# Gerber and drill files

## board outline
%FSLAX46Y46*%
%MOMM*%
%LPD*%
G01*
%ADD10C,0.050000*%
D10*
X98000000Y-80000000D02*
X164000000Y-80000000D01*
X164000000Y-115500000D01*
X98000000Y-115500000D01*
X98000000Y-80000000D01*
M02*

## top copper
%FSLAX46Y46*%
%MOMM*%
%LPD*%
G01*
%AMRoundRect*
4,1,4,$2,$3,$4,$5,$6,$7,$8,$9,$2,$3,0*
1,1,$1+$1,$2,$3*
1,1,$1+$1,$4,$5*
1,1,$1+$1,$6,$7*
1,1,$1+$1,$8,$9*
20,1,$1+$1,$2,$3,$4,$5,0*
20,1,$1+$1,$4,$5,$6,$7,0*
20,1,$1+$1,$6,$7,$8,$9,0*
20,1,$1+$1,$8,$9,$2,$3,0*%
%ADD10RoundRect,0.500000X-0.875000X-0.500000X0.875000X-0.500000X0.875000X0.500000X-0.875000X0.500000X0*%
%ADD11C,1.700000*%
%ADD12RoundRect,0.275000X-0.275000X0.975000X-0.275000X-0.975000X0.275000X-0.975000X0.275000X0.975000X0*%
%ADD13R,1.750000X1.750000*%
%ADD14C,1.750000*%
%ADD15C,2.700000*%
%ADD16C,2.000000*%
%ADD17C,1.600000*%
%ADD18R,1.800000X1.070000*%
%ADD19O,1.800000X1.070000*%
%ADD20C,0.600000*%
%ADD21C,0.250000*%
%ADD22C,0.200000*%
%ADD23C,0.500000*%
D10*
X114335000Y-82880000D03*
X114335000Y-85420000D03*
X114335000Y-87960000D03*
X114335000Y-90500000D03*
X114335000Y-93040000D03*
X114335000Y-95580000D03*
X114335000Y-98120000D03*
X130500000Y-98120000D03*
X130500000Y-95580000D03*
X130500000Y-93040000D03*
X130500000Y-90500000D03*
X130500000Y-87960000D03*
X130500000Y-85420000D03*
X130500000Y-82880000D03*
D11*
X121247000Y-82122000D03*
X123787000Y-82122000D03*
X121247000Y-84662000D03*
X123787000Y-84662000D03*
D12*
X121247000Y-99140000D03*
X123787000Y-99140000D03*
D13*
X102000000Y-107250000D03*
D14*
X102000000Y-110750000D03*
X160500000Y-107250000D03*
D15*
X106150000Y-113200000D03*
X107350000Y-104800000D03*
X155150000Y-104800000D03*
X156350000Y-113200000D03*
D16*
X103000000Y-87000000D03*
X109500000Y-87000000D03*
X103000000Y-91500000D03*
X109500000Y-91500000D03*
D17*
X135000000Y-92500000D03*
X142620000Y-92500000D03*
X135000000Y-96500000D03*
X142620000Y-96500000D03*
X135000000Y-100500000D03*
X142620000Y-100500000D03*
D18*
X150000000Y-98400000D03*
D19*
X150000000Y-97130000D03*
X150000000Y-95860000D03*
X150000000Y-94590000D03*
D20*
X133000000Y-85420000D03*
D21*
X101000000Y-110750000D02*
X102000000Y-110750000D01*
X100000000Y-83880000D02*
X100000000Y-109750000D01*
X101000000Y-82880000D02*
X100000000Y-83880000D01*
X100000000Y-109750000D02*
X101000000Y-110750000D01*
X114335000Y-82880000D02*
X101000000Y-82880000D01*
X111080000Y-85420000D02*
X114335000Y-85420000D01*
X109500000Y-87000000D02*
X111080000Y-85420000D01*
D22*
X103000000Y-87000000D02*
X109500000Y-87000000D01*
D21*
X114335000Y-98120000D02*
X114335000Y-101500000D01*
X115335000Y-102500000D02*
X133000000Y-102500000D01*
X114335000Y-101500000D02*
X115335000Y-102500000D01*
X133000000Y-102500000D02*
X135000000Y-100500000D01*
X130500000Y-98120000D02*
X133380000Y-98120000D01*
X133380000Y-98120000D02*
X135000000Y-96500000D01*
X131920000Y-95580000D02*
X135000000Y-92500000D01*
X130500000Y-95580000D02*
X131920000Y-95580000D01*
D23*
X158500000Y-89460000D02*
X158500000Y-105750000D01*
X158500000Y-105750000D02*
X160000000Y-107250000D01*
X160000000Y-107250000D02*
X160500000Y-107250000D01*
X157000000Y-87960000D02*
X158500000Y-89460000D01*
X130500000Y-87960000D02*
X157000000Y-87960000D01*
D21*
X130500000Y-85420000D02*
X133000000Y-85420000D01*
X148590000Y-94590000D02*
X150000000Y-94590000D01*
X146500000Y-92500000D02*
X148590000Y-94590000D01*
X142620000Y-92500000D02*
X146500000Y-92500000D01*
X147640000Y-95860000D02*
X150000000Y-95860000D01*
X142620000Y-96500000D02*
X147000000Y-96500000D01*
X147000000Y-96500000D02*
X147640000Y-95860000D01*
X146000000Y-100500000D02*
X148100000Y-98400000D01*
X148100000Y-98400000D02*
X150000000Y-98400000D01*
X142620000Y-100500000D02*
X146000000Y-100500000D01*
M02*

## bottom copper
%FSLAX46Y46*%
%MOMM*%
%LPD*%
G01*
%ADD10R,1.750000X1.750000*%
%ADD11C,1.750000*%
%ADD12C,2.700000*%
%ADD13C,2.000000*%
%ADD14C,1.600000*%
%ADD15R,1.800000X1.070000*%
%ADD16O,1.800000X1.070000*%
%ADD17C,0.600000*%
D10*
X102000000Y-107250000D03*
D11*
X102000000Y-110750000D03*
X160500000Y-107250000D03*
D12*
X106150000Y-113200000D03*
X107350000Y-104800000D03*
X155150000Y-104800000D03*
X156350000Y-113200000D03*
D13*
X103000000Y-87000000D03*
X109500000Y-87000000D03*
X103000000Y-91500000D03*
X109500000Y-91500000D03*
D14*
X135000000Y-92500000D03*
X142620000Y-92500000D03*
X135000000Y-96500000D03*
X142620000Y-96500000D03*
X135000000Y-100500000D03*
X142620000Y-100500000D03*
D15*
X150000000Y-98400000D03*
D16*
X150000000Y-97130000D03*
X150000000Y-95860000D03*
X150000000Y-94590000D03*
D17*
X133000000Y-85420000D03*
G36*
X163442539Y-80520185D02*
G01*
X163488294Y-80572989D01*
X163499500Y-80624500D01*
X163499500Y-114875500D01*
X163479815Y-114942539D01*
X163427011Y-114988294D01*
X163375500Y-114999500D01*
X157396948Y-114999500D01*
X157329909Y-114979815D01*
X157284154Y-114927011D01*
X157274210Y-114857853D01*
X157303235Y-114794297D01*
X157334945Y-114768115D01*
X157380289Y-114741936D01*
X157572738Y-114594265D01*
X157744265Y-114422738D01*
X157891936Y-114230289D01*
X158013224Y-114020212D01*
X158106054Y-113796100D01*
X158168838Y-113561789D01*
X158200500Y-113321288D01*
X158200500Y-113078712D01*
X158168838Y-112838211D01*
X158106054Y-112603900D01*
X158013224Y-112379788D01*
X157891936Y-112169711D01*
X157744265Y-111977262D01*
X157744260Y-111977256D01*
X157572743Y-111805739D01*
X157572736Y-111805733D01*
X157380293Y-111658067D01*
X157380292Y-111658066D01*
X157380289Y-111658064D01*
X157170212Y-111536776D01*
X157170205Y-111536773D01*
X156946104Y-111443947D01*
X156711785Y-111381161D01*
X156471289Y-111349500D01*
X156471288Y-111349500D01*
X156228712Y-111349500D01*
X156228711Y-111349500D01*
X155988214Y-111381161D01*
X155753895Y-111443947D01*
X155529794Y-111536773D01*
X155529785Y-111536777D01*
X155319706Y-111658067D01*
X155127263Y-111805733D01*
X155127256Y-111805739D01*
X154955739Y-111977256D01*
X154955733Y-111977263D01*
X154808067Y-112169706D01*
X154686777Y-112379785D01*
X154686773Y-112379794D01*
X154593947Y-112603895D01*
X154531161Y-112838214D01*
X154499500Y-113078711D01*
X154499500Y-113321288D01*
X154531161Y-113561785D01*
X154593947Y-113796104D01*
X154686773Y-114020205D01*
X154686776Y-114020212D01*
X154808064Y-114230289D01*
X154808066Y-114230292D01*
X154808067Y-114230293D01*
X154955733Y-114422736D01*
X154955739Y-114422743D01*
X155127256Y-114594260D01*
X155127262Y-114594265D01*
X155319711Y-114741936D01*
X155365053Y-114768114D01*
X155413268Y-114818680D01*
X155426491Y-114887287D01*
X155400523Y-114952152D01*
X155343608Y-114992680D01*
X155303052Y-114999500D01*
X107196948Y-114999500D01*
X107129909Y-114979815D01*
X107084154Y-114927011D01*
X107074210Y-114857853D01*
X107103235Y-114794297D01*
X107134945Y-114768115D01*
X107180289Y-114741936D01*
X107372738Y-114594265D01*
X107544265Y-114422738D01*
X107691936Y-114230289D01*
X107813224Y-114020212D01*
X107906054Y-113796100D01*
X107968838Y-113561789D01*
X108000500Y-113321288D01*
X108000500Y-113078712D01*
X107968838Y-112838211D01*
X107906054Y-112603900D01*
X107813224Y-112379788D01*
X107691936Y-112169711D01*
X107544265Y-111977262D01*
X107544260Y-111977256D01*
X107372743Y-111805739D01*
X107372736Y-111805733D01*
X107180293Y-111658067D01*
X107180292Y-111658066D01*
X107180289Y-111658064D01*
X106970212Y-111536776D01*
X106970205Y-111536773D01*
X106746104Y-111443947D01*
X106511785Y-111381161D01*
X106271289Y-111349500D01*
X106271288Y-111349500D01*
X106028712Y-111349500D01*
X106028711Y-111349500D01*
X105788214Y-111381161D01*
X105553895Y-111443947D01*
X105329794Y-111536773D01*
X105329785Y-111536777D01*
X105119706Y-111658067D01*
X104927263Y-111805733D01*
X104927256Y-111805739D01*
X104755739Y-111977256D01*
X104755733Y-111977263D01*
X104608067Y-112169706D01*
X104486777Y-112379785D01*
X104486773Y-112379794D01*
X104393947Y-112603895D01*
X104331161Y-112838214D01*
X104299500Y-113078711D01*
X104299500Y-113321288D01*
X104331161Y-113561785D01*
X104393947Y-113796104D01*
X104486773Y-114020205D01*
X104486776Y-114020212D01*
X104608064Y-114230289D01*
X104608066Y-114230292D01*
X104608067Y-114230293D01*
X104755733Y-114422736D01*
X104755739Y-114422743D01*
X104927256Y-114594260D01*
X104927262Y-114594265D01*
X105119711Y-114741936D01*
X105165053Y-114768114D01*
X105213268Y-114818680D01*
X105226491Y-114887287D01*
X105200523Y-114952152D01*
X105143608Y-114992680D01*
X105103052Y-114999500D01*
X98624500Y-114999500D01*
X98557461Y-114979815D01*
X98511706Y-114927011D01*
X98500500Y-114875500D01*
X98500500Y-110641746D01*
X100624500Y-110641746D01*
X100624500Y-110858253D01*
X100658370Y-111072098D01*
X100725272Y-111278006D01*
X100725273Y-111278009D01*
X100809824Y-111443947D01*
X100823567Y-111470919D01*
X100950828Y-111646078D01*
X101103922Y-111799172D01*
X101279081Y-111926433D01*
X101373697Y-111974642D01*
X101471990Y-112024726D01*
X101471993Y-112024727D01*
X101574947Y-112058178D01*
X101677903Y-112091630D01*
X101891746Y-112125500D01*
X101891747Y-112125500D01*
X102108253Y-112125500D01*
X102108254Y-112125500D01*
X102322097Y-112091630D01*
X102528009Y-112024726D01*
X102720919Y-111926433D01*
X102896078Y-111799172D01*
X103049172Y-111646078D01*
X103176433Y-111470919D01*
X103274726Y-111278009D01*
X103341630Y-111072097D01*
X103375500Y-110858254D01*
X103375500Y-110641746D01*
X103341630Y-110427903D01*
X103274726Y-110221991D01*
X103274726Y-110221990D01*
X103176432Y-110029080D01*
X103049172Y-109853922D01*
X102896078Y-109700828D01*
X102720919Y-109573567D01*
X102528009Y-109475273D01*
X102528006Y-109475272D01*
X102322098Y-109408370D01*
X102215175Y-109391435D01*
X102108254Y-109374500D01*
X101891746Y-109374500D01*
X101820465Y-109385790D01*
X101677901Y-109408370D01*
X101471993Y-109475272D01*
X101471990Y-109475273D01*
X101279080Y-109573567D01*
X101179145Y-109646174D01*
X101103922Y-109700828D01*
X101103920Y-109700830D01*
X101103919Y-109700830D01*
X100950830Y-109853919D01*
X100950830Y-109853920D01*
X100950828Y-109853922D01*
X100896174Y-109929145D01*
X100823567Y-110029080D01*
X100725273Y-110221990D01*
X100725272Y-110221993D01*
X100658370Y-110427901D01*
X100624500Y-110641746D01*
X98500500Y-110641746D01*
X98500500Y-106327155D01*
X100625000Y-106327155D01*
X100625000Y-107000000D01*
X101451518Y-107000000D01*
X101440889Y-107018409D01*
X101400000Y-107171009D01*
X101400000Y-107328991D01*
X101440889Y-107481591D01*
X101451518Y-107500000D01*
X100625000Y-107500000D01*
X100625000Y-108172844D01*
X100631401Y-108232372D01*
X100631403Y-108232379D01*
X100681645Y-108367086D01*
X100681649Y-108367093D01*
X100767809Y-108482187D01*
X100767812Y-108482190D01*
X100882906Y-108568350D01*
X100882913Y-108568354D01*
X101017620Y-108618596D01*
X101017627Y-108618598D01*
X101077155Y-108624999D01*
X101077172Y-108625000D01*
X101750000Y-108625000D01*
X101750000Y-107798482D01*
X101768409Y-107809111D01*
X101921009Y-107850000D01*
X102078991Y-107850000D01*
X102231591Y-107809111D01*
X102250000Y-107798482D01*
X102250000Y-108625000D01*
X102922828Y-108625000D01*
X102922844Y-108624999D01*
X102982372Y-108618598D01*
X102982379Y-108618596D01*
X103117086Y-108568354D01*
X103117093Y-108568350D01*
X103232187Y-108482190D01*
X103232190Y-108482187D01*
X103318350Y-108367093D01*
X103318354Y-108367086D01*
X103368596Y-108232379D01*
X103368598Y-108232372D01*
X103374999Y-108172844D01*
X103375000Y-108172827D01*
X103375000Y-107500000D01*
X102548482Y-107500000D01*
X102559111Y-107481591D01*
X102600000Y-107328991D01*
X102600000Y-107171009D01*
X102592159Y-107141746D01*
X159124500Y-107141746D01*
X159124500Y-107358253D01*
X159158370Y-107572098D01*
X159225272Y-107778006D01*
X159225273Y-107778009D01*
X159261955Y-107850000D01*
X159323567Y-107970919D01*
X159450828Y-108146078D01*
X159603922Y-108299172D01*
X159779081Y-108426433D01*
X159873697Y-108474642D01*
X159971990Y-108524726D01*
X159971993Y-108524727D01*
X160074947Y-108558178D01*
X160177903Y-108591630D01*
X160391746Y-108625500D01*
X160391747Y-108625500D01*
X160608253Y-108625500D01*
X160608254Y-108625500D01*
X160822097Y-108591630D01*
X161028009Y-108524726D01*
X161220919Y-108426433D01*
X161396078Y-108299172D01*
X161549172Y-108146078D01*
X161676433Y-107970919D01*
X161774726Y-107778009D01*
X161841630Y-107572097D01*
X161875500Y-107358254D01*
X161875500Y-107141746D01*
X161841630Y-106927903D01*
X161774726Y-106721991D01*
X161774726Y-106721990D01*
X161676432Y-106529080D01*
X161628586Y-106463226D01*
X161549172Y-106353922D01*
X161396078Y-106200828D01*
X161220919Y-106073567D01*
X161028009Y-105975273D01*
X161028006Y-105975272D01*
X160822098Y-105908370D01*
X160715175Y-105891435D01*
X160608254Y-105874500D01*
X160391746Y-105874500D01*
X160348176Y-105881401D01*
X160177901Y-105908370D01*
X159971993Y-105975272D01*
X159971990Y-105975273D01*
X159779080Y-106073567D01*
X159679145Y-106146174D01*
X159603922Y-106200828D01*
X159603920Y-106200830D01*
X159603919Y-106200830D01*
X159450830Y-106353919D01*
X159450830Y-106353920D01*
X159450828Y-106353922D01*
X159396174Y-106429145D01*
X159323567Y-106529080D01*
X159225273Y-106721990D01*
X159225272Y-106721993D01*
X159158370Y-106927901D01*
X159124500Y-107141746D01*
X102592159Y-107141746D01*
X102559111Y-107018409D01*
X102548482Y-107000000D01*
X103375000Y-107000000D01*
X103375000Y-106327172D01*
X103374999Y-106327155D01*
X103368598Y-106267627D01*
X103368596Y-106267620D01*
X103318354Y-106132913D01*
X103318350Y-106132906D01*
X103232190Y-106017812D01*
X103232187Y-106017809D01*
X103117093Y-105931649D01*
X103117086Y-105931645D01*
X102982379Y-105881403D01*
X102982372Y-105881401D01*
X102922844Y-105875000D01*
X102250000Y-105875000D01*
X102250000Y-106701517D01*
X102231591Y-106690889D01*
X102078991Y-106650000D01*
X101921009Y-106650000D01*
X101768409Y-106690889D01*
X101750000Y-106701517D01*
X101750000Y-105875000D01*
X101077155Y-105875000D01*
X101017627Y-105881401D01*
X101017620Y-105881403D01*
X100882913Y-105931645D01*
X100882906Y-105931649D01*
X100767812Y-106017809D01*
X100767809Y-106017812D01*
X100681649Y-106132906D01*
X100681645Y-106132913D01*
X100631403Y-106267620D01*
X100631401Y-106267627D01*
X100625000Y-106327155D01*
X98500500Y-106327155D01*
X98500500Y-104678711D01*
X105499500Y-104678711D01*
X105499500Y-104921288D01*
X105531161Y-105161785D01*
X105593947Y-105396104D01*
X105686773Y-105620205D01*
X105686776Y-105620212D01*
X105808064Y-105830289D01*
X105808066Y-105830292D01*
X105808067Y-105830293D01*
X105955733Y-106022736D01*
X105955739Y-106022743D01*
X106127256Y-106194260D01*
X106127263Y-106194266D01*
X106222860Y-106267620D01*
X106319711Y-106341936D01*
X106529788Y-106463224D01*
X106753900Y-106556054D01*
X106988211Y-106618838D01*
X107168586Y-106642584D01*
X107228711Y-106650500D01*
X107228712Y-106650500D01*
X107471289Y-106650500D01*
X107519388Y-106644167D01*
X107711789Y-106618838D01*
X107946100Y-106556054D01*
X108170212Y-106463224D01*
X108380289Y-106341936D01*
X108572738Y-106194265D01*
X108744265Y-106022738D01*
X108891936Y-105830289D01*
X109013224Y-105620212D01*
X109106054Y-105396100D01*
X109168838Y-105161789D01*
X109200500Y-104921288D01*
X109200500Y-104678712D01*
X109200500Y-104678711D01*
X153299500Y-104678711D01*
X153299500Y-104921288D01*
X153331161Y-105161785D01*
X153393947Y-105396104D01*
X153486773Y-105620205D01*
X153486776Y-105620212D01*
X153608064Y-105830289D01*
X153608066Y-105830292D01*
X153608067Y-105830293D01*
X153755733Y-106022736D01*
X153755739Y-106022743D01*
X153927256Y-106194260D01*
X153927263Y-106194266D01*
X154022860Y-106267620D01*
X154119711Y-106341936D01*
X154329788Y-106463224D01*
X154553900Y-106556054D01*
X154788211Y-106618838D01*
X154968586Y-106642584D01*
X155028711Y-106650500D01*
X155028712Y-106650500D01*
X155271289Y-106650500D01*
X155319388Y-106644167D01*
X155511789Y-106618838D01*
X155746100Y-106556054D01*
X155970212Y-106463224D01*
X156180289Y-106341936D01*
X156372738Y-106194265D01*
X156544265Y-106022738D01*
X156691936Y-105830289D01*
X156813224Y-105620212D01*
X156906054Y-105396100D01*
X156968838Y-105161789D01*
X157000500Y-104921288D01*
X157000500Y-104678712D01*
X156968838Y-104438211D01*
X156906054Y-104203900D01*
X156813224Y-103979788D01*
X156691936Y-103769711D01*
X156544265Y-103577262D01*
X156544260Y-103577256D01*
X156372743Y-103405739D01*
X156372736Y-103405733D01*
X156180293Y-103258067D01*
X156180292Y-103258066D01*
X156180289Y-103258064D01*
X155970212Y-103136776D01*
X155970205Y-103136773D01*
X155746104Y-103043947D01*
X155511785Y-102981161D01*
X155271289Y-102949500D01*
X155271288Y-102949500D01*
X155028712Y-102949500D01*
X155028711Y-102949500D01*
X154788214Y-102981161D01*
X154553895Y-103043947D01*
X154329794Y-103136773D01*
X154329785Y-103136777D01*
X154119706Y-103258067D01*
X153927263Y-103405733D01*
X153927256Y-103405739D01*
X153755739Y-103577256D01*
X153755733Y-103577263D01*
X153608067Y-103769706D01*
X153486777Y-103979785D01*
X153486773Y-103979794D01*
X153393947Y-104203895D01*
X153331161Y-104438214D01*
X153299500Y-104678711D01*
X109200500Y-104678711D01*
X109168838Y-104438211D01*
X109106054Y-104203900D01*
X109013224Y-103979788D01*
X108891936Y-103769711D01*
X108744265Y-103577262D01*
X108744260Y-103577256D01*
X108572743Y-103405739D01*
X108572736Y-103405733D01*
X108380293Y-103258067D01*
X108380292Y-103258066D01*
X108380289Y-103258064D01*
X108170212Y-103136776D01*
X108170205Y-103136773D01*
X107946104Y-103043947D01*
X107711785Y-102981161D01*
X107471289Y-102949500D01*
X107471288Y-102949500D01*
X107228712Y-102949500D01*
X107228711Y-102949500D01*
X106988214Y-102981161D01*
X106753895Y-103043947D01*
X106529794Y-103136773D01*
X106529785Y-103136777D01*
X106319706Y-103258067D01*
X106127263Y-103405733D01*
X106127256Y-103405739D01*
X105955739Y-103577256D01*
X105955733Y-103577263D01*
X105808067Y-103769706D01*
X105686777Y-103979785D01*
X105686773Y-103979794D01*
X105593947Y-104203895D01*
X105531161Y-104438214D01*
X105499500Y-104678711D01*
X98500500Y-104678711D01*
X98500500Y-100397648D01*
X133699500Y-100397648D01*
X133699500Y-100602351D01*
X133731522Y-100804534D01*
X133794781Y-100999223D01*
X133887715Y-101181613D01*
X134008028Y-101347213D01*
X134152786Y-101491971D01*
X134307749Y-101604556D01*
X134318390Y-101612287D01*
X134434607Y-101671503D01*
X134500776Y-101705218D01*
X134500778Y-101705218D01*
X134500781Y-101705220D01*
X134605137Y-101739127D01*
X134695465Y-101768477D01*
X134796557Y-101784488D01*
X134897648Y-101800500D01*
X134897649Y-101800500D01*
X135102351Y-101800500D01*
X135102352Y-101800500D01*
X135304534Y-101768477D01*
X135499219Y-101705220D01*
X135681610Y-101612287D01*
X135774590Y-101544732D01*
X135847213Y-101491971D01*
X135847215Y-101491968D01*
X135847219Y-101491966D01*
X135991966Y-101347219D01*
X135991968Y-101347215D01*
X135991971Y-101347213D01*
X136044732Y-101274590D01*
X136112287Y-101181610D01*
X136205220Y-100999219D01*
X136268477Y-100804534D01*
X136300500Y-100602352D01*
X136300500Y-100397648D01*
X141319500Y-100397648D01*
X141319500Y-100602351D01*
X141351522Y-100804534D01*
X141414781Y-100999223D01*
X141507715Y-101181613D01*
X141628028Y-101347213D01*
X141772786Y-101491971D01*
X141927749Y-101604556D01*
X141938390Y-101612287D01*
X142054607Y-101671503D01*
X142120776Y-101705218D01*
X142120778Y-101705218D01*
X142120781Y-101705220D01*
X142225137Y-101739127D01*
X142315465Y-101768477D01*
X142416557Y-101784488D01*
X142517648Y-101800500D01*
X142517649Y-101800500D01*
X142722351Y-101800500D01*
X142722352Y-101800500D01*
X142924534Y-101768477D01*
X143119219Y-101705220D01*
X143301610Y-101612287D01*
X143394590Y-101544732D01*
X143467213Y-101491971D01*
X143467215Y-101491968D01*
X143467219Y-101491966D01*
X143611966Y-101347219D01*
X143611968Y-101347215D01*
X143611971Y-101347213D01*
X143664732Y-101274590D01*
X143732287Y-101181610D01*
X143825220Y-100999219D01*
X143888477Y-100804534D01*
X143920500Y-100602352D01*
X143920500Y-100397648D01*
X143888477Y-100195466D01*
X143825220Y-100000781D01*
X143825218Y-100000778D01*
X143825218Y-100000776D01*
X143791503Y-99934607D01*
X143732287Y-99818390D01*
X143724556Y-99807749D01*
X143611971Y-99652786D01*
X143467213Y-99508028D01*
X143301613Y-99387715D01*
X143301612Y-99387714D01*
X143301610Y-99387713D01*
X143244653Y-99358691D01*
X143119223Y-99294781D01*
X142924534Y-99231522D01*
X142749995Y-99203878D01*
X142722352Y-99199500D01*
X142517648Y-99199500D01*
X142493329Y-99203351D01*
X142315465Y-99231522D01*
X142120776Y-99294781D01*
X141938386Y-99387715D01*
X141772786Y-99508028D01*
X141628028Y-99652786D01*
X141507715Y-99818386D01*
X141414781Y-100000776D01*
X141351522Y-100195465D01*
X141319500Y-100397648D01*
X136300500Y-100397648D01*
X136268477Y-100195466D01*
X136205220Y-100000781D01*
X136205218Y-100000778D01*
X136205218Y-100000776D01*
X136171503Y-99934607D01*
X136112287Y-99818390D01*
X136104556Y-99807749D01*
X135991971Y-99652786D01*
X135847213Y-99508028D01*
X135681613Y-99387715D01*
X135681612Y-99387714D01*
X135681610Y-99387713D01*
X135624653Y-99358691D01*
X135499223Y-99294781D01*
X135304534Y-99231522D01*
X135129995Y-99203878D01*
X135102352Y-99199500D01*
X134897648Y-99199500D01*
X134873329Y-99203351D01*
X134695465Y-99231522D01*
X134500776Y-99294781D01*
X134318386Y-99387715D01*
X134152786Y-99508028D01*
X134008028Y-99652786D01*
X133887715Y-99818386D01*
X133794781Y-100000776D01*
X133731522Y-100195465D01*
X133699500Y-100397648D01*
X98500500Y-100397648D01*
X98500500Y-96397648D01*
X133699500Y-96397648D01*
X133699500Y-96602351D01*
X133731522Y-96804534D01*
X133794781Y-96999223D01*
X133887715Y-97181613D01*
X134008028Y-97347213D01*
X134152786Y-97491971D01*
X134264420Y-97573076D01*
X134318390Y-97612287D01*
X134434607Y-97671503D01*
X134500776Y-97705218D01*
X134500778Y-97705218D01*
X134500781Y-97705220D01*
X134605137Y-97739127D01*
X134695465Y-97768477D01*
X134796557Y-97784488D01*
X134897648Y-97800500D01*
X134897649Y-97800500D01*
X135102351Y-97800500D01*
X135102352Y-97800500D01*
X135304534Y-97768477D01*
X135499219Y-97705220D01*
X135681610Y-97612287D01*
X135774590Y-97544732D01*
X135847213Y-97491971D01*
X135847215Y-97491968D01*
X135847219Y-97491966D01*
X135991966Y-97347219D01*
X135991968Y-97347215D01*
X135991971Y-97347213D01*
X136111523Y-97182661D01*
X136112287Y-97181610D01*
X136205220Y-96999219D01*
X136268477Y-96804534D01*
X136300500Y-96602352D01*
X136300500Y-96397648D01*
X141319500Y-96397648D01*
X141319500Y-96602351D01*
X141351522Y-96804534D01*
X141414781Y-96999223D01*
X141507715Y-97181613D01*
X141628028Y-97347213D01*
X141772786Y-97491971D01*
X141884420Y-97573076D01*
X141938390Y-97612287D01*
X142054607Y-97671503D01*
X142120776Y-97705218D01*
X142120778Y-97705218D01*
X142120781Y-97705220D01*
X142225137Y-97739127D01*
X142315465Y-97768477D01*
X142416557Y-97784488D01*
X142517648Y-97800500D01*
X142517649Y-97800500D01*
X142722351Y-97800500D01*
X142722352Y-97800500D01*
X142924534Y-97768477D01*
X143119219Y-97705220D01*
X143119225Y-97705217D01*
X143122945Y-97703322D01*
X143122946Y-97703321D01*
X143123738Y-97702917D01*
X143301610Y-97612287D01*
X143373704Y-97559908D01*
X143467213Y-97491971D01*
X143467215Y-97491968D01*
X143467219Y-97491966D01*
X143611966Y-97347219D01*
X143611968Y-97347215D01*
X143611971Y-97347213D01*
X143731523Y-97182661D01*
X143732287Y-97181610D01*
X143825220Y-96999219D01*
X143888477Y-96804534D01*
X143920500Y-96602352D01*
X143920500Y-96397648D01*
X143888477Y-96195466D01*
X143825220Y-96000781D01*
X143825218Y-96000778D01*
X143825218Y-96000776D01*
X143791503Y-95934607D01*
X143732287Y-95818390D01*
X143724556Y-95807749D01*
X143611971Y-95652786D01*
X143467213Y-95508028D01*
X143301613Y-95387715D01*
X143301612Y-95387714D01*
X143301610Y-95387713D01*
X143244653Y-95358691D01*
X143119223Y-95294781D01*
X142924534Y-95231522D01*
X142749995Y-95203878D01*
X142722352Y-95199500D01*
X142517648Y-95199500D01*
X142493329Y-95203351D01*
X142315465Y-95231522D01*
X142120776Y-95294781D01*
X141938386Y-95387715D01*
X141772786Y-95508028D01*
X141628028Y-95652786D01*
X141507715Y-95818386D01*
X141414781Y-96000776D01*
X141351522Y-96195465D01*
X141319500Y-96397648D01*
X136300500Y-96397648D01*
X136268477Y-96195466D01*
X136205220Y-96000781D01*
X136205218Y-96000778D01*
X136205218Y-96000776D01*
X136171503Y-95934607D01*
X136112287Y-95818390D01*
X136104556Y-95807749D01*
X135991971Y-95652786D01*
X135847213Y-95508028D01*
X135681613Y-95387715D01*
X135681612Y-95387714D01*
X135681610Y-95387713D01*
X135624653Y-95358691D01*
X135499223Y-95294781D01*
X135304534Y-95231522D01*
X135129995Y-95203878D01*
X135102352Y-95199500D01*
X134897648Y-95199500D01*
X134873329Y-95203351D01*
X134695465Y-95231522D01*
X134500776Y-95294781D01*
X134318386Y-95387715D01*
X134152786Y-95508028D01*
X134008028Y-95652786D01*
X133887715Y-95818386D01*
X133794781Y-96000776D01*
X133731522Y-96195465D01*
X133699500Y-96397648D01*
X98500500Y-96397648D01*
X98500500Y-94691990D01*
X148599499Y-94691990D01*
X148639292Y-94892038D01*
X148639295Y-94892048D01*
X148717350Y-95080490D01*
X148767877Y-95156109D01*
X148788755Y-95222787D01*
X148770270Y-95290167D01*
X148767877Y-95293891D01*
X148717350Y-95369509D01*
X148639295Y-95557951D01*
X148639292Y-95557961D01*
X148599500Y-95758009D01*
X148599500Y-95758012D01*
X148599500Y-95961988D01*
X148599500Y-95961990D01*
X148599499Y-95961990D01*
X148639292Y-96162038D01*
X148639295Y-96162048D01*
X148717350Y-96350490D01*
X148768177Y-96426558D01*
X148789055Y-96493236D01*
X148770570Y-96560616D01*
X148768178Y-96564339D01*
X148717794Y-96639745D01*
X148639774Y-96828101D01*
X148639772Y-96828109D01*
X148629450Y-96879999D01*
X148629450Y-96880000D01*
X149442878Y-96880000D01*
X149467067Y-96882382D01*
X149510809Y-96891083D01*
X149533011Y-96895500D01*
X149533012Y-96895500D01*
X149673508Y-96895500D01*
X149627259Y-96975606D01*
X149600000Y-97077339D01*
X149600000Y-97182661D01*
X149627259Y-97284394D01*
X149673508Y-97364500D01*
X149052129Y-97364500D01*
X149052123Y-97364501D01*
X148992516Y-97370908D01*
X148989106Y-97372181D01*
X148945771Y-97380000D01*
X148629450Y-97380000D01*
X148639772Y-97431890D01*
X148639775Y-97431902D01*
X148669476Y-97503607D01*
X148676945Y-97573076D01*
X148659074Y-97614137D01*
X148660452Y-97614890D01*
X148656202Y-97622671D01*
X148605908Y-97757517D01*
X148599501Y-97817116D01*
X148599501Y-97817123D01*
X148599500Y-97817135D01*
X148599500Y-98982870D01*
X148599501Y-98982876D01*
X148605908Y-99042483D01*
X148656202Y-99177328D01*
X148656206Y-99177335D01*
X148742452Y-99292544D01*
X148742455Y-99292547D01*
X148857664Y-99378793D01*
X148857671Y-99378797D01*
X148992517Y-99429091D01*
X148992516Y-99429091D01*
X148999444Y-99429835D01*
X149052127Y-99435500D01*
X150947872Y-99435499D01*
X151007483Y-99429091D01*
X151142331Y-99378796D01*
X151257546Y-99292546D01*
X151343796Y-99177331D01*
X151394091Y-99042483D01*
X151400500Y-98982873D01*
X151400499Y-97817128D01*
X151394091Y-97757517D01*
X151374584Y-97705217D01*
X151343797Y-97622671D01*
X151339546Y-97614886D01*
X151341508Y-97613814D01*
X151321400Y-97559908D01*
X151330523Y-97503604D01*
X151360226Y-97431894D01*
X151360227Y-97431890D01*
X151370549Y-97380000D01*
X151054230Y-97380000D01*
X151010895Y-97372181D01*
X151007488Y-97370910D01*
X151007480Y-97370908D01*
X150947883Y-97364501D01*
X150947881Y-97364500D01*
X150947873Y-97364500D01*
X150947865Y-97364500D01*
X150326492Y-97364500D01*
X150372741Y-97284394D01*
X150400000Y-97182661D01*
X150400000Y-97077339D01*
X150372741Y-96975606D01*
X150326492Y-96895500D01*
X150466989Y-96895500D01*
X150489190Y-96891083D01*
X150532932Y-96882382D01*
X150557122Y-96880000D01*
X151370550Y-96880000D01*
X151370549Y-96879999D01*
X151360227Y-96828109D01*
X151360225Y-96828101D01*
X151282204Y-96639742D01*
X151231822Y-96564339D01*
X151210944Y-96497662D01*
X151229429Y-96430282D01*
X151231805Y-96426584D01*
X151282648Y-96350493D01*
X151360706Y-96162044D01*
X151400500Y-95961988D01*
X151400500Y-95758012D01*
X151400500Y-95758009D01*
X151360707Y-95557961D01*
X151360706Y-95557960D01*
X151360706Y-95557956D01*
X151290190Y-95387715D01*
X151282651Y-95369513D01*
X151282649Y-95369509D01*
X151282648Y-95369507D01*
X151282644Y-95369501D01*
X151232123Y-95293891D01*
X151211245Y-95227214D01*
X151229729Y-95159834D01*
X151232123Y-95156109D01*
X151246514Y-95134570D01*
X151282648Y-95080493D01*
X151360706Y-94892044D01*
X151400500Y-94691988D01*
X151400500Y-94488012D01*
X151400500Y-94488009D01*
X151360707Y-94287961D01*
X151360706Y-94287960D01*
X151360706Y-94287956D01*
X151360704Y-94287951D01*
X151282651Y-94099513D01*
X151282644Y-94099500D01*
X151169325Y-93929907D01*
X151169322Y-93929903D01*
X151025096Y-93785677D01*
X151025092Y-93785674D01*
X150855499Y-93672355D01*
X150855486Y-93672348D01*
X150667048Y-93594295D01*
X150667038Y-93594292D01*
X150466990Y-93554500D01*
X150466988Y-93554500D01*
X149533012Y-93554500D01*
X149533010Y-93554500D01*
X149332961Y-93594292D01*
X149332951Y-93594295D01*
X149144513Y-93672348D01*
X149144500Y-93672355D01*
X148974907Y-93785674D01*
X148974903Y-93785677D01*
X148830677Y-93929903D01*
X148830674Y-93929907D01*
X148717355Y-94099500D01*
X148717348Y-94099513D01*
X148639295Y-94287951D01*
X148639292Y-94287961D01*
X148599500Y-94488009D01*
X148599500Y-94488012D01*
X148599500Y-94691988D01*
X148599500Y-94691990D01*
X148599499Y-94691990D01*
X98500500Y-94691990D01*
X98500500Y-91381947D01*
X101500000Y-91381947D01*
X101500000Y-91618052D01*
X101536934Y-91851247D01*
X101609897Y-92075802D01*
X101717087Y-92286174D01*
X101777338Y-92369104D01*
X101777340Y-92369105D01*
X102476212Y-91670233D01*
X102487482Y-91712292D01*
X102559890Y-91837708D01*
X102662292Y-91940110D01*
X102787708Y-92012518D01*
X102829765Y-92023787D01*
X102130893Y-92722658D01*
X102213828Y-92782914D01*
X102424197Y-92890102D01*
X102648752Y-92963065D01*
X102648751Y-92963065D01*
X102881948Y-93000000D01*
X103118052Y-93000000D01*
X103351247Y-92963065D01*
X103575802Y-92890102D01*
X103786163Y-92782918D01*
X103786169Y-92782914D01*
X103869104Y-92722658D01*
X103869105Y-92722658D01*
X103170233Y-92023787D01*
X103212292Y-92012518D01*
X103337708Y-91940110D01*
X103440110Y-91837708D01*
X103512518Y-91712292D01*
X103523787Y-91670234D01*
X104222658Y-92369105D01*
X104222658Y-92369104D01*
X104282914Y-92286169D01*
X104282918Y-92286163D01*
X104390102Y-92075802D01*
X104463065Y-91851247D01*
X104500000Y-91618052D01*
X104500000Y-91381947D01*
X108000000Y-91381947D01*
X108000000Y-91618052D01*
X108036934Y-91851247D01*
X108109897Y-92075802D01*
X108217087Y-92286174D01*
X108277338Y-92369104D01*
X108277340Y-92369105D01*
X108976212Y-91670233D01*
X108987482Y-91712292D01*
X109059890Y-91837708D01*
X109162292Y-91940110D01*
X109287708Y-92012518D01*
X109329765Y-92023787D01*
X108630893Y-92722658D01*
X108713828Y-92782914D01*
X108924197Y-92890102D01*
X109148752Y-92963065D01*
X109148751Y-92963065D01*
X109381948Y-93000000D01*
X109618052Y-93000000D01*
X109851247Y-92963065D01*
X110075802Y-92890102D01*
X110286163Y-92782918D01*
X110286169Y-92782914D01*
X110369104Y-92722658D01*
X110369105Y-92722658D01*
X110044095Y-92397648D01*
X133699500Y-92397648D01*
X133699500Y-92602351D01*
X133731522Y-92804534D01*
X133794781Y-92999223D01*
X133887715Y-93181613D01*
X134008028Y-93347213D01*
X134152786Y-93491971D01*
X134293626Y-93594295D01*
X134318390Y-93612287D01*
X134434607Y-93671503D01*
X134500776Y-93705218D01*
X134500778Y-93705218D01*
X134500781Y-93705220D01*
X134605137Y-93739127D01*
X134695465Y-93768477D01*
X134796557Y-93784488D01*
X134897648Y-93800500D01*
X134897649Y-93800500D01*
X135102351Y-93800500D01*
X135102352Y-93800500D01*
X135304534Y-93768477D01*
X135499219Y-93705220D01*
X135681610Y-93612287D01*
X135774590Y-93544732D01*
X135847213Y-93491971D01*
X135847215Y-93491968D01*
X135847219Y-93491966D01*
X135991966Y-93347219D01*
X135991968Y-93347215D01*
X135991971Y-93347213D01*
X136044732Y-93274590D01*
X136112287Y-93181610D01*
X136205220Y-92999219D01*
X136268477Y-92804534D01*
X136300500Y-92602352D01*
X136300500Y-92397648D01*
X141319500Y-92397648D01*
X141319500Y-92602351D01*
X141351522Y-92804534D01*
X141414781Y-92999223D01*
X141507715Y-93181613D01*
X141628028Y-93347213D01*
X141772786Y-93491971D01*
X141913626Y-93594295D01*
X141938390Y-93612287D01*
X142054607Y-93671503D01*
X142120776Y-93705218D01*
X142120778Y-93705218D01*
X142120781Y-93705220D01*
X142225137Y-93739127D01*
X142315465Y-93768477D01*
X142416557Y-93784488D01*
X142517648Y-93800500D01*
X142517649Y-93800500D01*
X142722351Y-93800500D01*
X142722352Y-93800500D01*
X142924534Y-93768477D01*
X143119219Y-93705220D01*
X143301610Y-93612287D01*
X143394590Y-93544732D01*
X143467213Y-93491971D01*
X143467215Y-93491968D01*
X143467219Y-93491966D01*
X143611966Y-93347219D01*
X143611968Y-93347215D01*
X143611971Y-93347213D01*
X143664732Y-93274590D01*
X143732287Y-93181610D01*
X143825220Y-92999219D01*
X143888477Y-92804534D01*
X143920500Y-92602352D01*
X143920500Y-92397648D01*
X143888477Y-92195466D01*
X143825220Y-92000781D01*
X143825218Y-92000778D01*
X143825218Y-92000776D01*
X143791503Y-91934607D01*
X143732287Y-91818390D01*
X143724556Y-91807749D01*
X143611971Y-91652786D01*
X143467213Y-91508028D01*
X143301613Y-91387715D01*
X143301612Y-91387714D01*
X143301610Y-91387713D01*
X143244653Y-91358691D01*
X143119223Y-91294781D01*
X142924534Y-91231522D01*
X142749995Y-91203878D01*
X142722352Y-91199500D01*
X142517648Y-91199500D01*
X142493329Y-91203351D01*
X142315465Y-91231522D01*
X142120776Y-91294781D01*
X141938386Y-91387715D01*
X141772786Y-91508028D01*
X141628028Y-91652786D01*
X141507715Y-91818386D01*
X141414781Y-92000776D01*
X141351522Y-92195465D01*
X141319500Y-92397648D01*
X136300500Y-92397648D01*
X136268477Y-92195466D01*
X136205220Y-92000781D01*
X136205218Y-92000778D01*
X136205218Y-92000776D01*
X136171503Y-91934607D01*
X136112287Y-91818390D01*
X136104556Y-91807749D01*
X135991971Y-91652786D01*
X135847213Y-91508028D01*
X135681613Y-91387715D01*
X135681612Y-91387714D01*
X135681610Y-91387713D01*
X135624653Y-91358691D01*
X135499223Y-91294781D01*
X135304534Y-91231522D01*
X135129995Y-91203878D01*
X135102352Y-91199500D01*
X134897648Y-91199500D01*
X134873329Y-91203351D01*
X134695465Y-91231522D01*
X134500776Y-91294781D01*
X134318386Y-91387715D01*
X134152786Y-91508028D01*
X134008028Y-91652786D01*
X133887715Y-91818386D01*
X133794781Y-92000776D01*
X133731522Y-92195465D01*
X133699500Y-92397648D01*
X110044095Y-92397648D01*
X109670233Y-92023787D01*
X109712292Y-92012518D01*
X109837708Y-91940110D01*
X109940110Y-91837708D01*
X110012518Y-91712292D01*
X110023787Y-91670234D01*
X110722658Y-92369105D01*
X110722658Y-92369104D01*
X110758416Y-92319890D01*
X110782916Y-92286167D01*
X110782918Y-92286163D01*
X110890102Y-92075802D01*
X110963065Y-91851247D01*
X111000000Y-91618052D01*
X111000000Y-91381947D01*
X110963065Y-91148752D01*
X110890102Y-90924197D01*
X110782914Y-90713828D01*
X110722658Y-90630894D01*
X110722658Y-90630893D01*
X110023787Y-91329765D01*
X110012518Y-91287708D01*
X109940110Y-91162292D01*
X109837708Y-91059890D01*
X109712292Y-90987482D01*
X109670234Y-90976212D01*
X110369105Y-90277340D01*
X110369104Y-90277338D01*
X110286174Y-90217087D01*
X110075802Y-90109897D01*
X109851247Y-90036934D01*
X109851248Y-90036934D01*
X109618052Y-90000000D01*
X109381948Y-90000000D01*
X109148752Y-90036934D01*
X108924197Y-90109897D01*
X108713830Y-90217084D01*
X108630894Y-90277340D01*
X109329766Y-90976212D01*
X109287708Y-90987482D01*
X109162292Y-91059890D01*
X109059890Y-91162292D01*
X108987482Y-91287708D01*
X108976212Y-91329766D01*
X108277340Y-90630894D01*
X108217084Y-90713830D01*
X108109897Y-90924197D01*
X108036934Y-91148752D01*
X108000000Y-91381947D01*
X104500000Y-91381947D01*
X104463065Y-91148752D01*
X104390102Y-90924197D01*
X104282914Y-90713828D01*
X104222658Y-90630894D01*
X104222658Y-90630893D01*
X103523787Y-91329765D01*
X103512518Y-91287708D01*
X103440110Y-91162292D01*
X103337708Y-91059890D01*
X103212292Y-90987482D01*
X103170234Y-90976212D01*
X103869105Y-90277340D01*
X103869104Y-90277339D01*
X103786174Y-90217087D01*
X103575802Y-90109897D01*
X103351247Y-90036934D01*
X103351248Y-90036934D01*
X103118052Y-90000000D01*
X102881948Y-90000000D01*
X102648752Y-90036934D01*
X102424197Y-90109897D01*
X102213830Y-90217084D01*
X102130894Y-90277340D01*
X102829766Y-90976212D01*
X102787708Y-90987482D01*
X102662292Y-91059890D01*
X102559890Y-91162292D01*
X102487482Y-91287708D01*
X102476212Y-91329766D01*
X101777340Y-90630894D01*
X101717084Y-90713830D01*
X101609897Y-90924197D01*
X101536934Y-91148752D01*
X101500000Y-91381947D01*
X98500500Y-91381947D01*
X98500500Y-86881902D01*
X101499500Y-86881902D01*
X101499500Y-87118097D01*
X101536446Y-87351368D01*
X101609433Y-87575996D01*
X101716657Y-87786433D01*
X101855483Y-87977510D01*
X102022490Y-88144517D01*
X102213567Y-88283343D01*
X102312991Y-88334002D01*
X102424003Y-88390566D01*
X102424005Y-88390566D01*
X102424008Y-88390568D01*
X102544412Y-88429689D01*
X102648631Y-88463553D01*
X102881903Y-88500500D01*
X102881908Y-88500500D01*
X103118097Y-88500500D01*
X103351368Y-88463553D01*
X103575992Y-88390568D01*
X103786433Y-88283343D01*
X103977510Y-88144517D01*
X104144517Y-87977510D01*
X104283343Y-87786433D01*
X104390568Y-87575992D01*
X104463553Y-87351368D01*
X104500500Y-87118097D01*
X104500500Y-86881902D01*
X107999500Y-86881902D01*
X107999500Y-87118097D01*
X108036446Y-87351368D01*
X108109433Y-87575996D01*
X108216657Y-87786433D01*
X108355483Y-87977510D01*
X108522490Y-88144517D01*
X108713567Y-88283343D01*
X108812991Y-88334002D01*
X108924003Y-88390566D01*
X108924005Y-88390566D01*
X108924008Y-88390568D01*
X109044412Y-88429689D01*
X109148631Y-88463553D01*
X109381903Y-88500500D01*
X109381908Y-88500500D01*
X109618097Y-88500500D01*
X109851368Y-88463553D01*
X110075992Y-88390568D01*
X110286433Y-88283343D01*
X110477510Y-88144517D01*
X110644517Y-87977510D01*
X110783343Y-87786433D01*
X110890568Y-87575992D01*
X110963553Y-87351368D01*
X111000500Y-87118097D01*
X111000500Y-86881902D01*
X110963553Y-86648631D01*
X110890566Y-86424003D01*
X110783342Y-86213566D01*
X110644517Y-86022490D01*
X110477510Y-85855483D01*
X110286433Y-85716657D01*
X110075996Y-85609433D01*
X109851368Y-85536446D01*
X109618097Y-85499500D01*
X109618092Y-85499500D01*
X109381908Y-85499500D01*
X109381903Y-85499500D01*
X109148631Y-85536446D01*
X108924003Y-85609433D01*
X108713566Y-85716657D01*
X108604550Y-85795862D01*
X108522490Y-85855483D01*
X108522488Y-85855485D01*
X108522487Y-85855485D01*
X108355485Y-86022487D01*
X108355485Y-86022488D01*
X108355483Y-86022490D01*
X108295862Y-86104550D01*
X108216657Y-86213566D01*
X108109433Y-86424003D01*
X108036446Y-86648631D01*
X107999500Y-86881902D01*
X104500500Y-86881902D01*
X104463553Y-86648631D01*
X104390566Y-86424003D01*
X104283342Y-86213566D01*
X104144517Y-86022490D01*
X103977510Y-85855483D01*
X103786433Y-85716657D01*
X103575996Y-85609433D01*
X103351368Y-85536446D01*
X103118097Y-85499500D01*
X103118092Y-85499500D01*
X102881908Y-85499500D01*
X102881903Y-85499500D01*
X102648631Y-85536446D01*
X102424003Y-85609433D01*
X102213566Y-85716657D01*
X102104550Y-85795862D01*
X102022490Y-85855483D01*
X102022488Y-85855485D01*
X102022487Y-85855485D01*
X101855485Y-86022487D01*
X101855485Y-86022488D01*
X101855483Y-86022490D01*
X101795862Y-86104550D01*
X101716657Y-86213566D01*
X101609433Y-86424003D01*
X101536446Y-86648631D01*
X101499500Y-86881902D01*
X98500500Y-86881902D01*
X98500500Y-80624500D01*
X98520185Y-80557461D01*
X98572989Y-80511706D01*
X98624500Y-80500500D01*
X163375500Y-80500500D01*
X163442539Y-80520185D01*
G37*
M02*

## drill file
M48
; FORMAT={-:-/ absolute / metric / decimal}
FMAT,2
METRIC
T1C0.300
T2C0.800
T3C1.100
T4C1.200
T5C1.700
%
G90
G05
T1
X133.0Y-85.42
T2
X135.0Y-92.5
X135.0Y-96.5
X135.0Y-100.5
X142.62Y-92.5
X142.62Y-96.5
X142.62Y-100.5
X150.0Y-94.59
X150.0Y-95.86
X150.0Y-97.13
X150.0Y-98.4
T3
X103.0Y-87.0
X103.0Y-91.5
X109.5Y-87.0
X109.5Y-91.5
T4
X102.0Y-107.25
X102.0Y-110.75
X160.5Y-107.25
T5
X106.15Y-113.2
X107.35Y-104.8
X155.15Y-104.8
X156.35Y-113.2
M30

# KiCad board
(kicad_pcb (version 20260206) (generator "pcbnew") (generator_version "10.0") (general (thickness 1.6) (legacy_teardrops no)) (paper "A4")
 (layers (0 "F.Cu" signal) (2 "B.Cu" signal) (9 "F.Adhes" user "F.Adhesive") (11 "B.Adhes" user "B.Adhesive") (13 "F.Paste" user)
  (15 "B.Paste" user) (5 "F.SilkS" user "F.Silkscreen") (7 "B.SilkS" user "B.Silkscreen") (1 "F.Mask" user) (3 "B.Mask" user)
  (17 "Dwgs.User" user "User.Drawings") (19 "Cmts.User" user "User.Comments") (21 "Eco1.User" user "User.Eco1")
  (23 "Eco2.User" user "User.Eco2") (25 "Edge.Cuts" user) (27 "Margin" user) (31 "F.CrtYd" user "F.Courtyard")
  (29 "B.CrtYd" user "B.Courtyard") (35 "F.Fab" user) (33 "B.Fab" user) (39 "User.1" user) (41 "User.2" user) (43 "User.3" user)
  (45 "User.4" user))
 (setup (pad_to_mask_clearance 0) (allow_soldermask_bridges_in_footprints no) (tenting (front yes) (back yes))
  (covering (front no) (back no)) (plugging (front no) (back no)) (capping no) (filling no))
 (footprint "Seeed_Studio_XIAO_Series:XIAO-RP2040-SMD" (layer "F.Cu") (at 113.5 101)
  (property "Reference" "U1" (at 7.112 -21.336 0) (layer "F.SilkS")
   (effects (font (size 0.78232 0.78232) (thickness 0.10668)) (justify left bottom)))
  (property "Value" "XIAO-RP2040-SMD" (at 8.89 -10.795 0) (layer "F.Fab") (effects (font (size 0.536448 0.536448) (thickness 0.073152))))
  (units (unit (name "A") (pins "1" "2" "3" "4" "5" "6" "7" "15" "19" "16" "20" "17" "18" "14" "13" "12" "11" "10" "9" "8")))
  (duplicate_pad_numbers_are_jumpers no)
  (pad "1" smd roundrect (at 0.835 -18.12) (size 2.75 2) (layers "F.Cu" "F.Mask" "F.Paste") (roundrect_rratio 0.25) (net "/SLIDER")
   (solder_mask_margin 0.0508) (thermal_bridge_angle 45))
  (pad "2" smd roundrect (at 0.835 -15.58) (size 2.75 2) (layers "F.Cu" "F.Mask" "F.Paste") (roundrect_rratio 0.25) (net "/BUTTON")
   (solder_mask_margin 0.0508) (thermal_bridge_angle 45))
  (pad "3" smd roundrect (at 0.835 -13.04) (size 2.75 2) (layers "F.Cu" "F.Mask" "F.Paste") (roundrect_rratio 0.25)
   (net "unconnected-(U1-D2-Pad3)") (solder_mask_margin 0.0508) (thermal_bridge_angle 45))
  (pad "4" smd roundrect (at 0.835 -10.5) (size 2.75 2) (layers "F.Cu" "F.Mask" "F.Paste") (roundrect_rratio 0.25)
   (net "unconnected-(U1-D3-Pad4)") (solder_mask_margin 0.0508) (thermal_bridge_angle 45))
  (pad "5" smd roundrect (at 0.835 -7.96) (size 2.75 2) (layers "F.Cu" "F.Mask" "F.Paste") (roundrect_rratio 0.25)
   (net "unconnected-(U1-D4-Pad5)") (solder_mask_margin 0.0508) (thermal_bridge_angle 45))
  (pad "6" smd roundrect (at 0.835 -5.42) (size 2.75 2) (layers "F.Cu" "F.Mask" "F.Paste") (roundrect_rratio 0.25)
   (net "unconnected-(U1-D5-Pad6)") (solder_mask_margin 0.0508) (thermal_bridge_angle 45))
  (pad "7" smd roundrect (at 0.835 -2.88) (size 2.75 2) (layers "F.Cu" "F.Mask" "F.Paste") (roundrect_rratio 0.25) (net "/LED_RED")
   (solder_mask_margin 0.0508) (thermal_bridge_angle 45))
  (pad "8" smd roundrect (at 17 -2.88) (size 2.75 2) (layers "F.Cu" "F.Mask" "F.Paste") (roundrect_rratio 0.25) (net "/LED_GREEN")
   (solder_mask_margin 0.0508) (thermal_bridge_angle 45))
  (pad "9" smd roundrect (at 17 -5.42) (size 2.75 2) (layers "F.Cu" "F.Mask" "F.Paste") (roundrect_rratio 0.25) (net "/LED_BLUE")
   (solder_mask_margin 0.0508) (thermal_bridge_angle 45))
  (pad "10" smd roundrect (at 17 -7.96) (size 2.75 2) (layers "F.Cu" "F.Mask" "F.Paste") (roundrect_rratio 0.25)
   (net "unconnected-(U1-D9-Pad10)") (solder_mask_margin 0.0508) (thermal_bridge_angle 45))
  (pad "11" smd roundrect (at 17 -10.5) (size 2.75 2) (layers "F.Cu" "F.Mask" "F.Paste") (roundrect_rratio 0.25)
   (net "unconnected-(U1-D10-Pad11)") (solder_mask_margin 0.0508) (thermal_bridge_angle 45))
  (pad "12" smd roundrect (at 17 -13.04) (size 2.75 2) (layers "F.Cu" "F.Mask" "F.Paste") (roundrect_rratio 0.25) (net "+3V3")
   (solder_mask_margin 0.0508) (thermal_bridge_angle 45))
  (pad "13" smd roundrect (at 17 -15.58) (size 2.75 2) (layers "F.Cu" "F.Mask" "F.Paste") (roundrect_rratio 0.25) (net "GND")
   (solder_mask_margin 0.0508) (thermal_bridge_angle 45))
  (pad "14" smd roundrect (at 17 -18.12) (size 2.75 2) (layers "F.Cu" "F.Mask" "F.Paste") (roundrect_rratio 0.25)
   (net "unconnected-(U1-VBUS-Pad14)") (solder_mask_margin 0.0508) (thermal_bridge_angle 45))
  (pad "15" smd circle (at 7.747 -18.878) (size 1.7 1.7) (layers "F.Cu" "F.Mask" "F.Paste") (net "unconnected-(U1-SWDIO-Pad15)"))
  (pad "16" smd circle (at 10.287 -18.878) (size 1.7 1.7) (layers "F.Cu" "F.Mask" "F.Paste") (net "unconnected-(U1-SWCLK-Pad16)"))
  (pad "17" smd circle (at 7.747 -16.338) (size 1.7 1.7) (layers "F.Cu" "F.Mask" "F.Paste") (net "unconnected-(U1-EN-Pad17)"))
  (pad "18" smd circle (at 10.287 -16.338) (size 1.7 1.7) (layers "F.Cu" "F.Mask" "F.Paste") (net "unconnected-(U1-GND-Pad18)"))
  (pad "19" smd roundrect (at 7.747 -1.86 270) (size 2.5 1.1) (layers "F.Cu" "F.Mask" "F.Paste") (roundrect_rratio 0.25)
   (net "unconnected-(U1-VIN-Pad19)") (thermal_bridge_angle 45))
  (pad "20" smd roundrect (at 10.287 -1.86 270) (size 2.5 1.1) (layers "F.Cu" "F.Mask" "F.Paste") (roundrect_rratio 0.25)
   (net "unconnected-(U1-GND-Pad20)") (thermal_bridge_angle 45)))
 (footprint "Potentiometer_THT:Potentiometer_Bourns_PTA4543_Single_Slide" (layer "F.Cu") (at 102 107.25)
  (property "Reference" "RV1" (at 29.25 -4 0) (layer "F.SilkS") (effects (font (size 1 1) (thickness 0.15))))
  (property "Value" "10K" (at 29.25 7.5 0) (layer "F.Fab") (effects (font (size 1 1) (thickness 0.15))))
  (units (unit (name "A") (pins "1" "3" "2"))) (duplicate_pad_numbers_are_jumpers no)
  (pad "1" thru_hole rect (at 0 0) (size 1.75 1.75) (drill 1.2) (layers "*.Cu" "*.Mask") (remove_unused_layers no) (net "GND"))
  (pad "2" thru_hole circle (at 0 3.5) (size 1.75 1.75) (drill 1.2) (layers "*.Cu" "*.Mask") (remove_unused_layers no) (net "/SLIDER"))
  (pad "3" thru_hole circle (at 58.5 0) (size 1.75 1.75) (drill 1.2) (layers "*.Cu" "*.Mask") (remove_unused_layers no) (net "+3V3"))
  (pad "MP" thru_hole circle (at 4.15 5.95) (size 2.7 2.7) (drill 1.7) (layers "*.Cu" "*.Mask") (remove_unused_layers no))
  (pad "MP" thru_hole circle (at 5.35 -2.45) (size 2.7 2.7) (drill 1.7) (layers "*.Cu" "*.Mask") (remove_unused_layers no))
  (pad "MP" thru_hole circle (at 53.15 -2.45) (size 2.7 2.7) (drill 1.7) (layers "*.Cu" "*.Mask") (remove_unused_layers no))
  (pad "MP" thru_hole circle (at 54.35 5.95) (size 2.7 2.7) (drill 1.7) (layers "*.Cu" "*.Mask") (remove_unused_layers no)))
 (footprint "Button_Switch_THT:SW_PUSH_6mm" (layer "F.Cu") (at 103 87)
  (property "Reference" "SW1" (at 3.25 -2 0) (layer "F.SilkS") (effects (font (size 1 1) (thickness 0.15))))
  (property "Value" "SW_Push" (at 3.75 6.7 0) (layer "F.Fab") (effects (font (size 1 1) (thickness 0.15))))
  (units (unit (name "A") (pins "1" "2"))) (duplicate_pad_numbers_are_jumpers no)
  (pad "1" thru_hole circle (at 0 0 90) (size 2 2) (drill 1.1) (layers "*.Cu" "*.Mask") (remove_unused_layers no) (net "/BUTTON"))
  (pad "1" thru_hole circle (at 6.5 0 90) (size 2 2) (drill 1.1) (layers "*.Cu" "*.Mask") (remove_unused_layers no) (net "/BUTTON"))
  (pad "2" thru_hole circle (at 0 4.5 90) (size 2 2) (drill 1.1) (layers "*.Cu" "*.Mask") (remove_unused_layers no) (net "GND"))
  (pad "2" thru_hole circle (at 6.5 4.5 90) (size 2 2) (drill 1.1) (layers "*.Cu" "*.Mask") (remove_unused_layers no) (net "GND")))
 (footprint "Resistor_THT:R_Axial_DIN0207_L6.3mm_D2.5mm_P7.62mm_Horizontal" (layer "F.Cu") (at 135 92.5)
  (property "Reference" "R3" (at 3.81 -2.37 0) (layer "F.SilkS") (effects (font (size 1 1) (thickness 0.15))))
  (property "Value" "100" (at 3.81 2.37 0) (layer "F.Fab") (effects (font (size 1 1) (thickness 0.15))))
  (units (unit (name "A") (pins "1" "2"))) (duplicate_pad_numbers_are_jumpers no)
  (pad "1" thru_hole circle (at 0 0) (size 1.6 1.6) (drill 0.8) (layers "*.Cu" "*.Mask") (remove_unused_layers no) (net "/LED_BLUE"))
  (pad "2" thru_hole circle (at 7.62 0) (size 1.6 1.6) (drill 0.8) (layers "*.Cu" "*.Mask") (remove_unused_layers no) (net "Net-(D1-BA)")))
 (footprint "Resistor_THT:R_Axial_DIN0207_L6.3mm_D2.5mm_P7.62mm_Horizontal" (layer "F.Cu") (at 135 96.5)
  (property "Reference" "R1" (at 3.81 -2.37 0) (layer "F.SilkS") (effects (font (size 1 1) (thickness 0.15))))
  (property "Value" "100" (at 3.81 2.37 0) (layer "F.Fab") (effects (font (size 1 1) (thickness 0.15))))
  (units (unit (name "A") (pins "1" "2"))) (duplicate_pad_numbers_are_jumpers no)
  (pad "1" thru_hole circle (at 0 0) (size 1.6 1.6) (drill 0.8) (layers "*.Cu" "*.Mask") (remove_unused_layers no) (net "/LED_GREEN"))
  (pad "2" thru_hole circle (at 7.62 0) (size 1.6 1.6) (drill 0.8) (layers "*.Cu" "*.Mask") (remove_unused_layers no) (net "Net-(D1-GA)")))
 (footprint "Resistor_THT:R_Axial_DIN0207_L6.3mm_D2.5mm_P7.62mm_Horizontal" (layer "F.Cu") (at 135 100.5)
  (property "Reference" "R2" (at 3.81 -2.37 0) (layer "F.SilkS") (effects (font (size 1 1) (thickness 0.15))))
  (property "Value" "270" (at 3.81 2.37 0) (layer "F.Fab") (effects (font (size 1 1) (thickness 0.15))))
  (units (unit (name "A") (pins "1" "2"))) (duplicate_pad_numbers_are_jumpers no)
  (pad "1" thru_hole circle (at 0 0) (size 1.6 1.6) (drill 0.8) (layers "*.Cu" "*.Mask") (remove_unused_layers no) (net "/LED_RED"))
  (pad "2" thru_hole circle (at 7.62 0) (size 1.6 1.6) (drill 0.8) (layers "*.Cu" "*.Mask") (remove_unused_layers no) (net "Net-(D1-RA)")))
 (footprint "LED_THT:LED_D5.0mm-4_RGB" (layer "F.Cu") (at 150 98.4 90)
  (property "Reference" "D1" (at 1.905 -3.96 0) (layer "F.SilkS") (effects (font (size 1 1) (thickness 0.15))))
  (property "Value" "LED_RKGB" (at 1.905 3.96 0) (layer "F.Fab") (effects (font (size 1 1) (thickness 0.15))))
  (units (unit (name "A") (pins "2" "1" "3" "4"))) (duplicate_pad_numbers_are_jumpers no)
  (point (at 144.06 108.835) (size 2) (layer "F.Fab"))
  (pad "1" thru_hole rect (at 0 0 90) (size 1.07 1.8) (drill 0.8) (layers "*.Cu" "*.Mask") (remove_unused_layers no) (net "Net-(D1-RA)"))
  (pad "2" thru_hole oval (at 1.27 0 90) (size 1.07 1.8) (drill 0.8) (layers "*.Cu" "*.Mask") (remove_unused_layers no) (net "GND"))
  (pad "3" thru_hole oval (at 2.54 0 90) (size 1.07 1.8) (drill 0.8) (layers "*.Cu" "*.Mask" "Dwgs.User") (remove_unused_layers no)
   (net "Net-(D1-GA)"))
  (pad "4" thru_hole oval (at 3.81 0 90) (size 1.07 1.8) (drill 0.8) (layers "*.Cu" "*.Mask") (remove_unused_layers no) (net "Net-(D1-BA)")))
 (gr_rect (start 98 80) (end 164 115.5) (stroke (width 0.05) (type default)) (fill no) (layer "Edge.Cuts"))
 (segment (start 101 110.75) (end 102 110.75) (width 0.25) (layer "F.Cu") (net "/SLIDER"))
 (segment (start 100 83.88) (end 100 109.75) (width 0.25) (layer "F.Cu") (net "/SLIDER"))
 (segment (start 101 82.88) (end 100 83.88) (width 0.25) (layer "F.Cu") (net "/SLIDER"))
 (segment (start 100 109.75) (end 101 110.75) (width 0.25) (layer "F.Cu") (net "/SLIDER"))
 (segment (start 114.335 82.88) (end 101 82.88) (width 0.25) (layer "F.Cu") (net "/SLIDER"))
 (segment (start 111.08 85.42) (end 114.335 85.42) (width 0.25) (layer "F.Cu") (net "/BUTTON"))
 (segment (start 109.5 87) (end 111.08 85.42) (width 0.25) (layer "F.Cu") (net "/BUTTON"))
 (segment (start 103 87) (end 109.5 87) (width 0.2) (layer "F.Cu") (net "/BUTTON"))
 (segment (start 114.335 98.12) (end 114.335 101.5) (width 0.25) (layer "F.Cu") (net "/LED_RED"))
 (segment (start 115.335 102.5) (end 133 102.5) (width 0.25) (layer "F.Cu") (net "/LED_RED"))
 (segment (start 114.335 101.5) (end 115.335 102.5) (width 0.25) (layer "F.Cu") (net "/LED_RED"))
 (segment (start 133 102.5) (end 135 100.5) (width 0.25) (layer "F.Cu") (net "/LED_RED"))
 (segment (start 130.5 98.12) (end 133.38 98.12) (width 0.25) (layer "F.Cu") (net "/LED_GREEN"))
 (segment (start 133.38 98.12) (end 135 96.5) (width 0.25) (layer "F.Cu") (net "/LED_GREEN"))
 (segment (start 131.92 95.58) (end 135 92.5) (width 0.25) (layer "F.Cu") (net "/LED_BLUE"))
 (segment (start 130.5 95.58) (end 131.92 95.58) (width 0.25) (layer "F.Cu") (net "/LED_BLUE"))
 (segment (start 158.5 89.46) (end 158.5 105.75) (width 0.5) (layer "F.Cu") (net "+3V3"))
 (segment (start 158.5 105.75) (end 160 107.25) (width 0.5) (layer "F.Cu") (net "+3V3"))
 (segment (start 160 107.25) (end 160.5 107.25) (width 0.5) (layer "F.Cu") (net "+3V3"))
 (segment (start 157 87.96) (end 158.5 89.46) (width 0.5) (layer "F.Cu") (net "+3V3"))
 (segment (start 130.5 87.96) (end 157 87.96) (width 0.5) (layer "F.Cu") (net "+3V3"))
 (segment (start 130.5 85.42) (end 133 85.42) (width 0.25) (layer "F.Cu") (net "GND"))
 (via (at 133 85.42) (size 0.6) (drill 0.3) (layers "F.Cu" "B.Cu") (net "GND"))
 (segment (start 148.59 94.59) (end 150 94.59) (width 0.25) (layer "F.Cu") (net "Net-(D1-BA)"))
 (segment (start 146.5 92.5) (end 148.59 94.59) (width 0.25) (layer "F.Cu") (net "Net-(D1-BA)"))
 (segment (start 142.62 92.5) (end 146.5 92.5) (width 0.25) (layer "F.Cu") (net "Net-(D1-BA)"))
 (segment (start 147.64 95.86) (end 150 95.86) (width 0.25) (layer "F.Cu") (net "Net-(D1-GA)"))
 (segment (start 142.62 96.5) (end 147 96.5) (width 0.25) (layer "F.Cu") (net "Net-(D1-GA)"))
 (segment (start 147 96.5) (end 147.64 95.86) (width 0.25) (layer "F.Cu") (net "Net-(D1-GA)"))
 (segment (start 146 100.5) (end 148.1 98.4) (width 0.25) (layer "F.Cu") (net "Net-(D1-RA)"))
 (segment (start 148.1 98.4) (end 150 98.4) (width 0.25) (layer "F.Cu") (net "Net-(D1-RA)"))
 (segment (start 142.62 100.5) (end 146 100.5) (width 0.25) (layer "F.Cu") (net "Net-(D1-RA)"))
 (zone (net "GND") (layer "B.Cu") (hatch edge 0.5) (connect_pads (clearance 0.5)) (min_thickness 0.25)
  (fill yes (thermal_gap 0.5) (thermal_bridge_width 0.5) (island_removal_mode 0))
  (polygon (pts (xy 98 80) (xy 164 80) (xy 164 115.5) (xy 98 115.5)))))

